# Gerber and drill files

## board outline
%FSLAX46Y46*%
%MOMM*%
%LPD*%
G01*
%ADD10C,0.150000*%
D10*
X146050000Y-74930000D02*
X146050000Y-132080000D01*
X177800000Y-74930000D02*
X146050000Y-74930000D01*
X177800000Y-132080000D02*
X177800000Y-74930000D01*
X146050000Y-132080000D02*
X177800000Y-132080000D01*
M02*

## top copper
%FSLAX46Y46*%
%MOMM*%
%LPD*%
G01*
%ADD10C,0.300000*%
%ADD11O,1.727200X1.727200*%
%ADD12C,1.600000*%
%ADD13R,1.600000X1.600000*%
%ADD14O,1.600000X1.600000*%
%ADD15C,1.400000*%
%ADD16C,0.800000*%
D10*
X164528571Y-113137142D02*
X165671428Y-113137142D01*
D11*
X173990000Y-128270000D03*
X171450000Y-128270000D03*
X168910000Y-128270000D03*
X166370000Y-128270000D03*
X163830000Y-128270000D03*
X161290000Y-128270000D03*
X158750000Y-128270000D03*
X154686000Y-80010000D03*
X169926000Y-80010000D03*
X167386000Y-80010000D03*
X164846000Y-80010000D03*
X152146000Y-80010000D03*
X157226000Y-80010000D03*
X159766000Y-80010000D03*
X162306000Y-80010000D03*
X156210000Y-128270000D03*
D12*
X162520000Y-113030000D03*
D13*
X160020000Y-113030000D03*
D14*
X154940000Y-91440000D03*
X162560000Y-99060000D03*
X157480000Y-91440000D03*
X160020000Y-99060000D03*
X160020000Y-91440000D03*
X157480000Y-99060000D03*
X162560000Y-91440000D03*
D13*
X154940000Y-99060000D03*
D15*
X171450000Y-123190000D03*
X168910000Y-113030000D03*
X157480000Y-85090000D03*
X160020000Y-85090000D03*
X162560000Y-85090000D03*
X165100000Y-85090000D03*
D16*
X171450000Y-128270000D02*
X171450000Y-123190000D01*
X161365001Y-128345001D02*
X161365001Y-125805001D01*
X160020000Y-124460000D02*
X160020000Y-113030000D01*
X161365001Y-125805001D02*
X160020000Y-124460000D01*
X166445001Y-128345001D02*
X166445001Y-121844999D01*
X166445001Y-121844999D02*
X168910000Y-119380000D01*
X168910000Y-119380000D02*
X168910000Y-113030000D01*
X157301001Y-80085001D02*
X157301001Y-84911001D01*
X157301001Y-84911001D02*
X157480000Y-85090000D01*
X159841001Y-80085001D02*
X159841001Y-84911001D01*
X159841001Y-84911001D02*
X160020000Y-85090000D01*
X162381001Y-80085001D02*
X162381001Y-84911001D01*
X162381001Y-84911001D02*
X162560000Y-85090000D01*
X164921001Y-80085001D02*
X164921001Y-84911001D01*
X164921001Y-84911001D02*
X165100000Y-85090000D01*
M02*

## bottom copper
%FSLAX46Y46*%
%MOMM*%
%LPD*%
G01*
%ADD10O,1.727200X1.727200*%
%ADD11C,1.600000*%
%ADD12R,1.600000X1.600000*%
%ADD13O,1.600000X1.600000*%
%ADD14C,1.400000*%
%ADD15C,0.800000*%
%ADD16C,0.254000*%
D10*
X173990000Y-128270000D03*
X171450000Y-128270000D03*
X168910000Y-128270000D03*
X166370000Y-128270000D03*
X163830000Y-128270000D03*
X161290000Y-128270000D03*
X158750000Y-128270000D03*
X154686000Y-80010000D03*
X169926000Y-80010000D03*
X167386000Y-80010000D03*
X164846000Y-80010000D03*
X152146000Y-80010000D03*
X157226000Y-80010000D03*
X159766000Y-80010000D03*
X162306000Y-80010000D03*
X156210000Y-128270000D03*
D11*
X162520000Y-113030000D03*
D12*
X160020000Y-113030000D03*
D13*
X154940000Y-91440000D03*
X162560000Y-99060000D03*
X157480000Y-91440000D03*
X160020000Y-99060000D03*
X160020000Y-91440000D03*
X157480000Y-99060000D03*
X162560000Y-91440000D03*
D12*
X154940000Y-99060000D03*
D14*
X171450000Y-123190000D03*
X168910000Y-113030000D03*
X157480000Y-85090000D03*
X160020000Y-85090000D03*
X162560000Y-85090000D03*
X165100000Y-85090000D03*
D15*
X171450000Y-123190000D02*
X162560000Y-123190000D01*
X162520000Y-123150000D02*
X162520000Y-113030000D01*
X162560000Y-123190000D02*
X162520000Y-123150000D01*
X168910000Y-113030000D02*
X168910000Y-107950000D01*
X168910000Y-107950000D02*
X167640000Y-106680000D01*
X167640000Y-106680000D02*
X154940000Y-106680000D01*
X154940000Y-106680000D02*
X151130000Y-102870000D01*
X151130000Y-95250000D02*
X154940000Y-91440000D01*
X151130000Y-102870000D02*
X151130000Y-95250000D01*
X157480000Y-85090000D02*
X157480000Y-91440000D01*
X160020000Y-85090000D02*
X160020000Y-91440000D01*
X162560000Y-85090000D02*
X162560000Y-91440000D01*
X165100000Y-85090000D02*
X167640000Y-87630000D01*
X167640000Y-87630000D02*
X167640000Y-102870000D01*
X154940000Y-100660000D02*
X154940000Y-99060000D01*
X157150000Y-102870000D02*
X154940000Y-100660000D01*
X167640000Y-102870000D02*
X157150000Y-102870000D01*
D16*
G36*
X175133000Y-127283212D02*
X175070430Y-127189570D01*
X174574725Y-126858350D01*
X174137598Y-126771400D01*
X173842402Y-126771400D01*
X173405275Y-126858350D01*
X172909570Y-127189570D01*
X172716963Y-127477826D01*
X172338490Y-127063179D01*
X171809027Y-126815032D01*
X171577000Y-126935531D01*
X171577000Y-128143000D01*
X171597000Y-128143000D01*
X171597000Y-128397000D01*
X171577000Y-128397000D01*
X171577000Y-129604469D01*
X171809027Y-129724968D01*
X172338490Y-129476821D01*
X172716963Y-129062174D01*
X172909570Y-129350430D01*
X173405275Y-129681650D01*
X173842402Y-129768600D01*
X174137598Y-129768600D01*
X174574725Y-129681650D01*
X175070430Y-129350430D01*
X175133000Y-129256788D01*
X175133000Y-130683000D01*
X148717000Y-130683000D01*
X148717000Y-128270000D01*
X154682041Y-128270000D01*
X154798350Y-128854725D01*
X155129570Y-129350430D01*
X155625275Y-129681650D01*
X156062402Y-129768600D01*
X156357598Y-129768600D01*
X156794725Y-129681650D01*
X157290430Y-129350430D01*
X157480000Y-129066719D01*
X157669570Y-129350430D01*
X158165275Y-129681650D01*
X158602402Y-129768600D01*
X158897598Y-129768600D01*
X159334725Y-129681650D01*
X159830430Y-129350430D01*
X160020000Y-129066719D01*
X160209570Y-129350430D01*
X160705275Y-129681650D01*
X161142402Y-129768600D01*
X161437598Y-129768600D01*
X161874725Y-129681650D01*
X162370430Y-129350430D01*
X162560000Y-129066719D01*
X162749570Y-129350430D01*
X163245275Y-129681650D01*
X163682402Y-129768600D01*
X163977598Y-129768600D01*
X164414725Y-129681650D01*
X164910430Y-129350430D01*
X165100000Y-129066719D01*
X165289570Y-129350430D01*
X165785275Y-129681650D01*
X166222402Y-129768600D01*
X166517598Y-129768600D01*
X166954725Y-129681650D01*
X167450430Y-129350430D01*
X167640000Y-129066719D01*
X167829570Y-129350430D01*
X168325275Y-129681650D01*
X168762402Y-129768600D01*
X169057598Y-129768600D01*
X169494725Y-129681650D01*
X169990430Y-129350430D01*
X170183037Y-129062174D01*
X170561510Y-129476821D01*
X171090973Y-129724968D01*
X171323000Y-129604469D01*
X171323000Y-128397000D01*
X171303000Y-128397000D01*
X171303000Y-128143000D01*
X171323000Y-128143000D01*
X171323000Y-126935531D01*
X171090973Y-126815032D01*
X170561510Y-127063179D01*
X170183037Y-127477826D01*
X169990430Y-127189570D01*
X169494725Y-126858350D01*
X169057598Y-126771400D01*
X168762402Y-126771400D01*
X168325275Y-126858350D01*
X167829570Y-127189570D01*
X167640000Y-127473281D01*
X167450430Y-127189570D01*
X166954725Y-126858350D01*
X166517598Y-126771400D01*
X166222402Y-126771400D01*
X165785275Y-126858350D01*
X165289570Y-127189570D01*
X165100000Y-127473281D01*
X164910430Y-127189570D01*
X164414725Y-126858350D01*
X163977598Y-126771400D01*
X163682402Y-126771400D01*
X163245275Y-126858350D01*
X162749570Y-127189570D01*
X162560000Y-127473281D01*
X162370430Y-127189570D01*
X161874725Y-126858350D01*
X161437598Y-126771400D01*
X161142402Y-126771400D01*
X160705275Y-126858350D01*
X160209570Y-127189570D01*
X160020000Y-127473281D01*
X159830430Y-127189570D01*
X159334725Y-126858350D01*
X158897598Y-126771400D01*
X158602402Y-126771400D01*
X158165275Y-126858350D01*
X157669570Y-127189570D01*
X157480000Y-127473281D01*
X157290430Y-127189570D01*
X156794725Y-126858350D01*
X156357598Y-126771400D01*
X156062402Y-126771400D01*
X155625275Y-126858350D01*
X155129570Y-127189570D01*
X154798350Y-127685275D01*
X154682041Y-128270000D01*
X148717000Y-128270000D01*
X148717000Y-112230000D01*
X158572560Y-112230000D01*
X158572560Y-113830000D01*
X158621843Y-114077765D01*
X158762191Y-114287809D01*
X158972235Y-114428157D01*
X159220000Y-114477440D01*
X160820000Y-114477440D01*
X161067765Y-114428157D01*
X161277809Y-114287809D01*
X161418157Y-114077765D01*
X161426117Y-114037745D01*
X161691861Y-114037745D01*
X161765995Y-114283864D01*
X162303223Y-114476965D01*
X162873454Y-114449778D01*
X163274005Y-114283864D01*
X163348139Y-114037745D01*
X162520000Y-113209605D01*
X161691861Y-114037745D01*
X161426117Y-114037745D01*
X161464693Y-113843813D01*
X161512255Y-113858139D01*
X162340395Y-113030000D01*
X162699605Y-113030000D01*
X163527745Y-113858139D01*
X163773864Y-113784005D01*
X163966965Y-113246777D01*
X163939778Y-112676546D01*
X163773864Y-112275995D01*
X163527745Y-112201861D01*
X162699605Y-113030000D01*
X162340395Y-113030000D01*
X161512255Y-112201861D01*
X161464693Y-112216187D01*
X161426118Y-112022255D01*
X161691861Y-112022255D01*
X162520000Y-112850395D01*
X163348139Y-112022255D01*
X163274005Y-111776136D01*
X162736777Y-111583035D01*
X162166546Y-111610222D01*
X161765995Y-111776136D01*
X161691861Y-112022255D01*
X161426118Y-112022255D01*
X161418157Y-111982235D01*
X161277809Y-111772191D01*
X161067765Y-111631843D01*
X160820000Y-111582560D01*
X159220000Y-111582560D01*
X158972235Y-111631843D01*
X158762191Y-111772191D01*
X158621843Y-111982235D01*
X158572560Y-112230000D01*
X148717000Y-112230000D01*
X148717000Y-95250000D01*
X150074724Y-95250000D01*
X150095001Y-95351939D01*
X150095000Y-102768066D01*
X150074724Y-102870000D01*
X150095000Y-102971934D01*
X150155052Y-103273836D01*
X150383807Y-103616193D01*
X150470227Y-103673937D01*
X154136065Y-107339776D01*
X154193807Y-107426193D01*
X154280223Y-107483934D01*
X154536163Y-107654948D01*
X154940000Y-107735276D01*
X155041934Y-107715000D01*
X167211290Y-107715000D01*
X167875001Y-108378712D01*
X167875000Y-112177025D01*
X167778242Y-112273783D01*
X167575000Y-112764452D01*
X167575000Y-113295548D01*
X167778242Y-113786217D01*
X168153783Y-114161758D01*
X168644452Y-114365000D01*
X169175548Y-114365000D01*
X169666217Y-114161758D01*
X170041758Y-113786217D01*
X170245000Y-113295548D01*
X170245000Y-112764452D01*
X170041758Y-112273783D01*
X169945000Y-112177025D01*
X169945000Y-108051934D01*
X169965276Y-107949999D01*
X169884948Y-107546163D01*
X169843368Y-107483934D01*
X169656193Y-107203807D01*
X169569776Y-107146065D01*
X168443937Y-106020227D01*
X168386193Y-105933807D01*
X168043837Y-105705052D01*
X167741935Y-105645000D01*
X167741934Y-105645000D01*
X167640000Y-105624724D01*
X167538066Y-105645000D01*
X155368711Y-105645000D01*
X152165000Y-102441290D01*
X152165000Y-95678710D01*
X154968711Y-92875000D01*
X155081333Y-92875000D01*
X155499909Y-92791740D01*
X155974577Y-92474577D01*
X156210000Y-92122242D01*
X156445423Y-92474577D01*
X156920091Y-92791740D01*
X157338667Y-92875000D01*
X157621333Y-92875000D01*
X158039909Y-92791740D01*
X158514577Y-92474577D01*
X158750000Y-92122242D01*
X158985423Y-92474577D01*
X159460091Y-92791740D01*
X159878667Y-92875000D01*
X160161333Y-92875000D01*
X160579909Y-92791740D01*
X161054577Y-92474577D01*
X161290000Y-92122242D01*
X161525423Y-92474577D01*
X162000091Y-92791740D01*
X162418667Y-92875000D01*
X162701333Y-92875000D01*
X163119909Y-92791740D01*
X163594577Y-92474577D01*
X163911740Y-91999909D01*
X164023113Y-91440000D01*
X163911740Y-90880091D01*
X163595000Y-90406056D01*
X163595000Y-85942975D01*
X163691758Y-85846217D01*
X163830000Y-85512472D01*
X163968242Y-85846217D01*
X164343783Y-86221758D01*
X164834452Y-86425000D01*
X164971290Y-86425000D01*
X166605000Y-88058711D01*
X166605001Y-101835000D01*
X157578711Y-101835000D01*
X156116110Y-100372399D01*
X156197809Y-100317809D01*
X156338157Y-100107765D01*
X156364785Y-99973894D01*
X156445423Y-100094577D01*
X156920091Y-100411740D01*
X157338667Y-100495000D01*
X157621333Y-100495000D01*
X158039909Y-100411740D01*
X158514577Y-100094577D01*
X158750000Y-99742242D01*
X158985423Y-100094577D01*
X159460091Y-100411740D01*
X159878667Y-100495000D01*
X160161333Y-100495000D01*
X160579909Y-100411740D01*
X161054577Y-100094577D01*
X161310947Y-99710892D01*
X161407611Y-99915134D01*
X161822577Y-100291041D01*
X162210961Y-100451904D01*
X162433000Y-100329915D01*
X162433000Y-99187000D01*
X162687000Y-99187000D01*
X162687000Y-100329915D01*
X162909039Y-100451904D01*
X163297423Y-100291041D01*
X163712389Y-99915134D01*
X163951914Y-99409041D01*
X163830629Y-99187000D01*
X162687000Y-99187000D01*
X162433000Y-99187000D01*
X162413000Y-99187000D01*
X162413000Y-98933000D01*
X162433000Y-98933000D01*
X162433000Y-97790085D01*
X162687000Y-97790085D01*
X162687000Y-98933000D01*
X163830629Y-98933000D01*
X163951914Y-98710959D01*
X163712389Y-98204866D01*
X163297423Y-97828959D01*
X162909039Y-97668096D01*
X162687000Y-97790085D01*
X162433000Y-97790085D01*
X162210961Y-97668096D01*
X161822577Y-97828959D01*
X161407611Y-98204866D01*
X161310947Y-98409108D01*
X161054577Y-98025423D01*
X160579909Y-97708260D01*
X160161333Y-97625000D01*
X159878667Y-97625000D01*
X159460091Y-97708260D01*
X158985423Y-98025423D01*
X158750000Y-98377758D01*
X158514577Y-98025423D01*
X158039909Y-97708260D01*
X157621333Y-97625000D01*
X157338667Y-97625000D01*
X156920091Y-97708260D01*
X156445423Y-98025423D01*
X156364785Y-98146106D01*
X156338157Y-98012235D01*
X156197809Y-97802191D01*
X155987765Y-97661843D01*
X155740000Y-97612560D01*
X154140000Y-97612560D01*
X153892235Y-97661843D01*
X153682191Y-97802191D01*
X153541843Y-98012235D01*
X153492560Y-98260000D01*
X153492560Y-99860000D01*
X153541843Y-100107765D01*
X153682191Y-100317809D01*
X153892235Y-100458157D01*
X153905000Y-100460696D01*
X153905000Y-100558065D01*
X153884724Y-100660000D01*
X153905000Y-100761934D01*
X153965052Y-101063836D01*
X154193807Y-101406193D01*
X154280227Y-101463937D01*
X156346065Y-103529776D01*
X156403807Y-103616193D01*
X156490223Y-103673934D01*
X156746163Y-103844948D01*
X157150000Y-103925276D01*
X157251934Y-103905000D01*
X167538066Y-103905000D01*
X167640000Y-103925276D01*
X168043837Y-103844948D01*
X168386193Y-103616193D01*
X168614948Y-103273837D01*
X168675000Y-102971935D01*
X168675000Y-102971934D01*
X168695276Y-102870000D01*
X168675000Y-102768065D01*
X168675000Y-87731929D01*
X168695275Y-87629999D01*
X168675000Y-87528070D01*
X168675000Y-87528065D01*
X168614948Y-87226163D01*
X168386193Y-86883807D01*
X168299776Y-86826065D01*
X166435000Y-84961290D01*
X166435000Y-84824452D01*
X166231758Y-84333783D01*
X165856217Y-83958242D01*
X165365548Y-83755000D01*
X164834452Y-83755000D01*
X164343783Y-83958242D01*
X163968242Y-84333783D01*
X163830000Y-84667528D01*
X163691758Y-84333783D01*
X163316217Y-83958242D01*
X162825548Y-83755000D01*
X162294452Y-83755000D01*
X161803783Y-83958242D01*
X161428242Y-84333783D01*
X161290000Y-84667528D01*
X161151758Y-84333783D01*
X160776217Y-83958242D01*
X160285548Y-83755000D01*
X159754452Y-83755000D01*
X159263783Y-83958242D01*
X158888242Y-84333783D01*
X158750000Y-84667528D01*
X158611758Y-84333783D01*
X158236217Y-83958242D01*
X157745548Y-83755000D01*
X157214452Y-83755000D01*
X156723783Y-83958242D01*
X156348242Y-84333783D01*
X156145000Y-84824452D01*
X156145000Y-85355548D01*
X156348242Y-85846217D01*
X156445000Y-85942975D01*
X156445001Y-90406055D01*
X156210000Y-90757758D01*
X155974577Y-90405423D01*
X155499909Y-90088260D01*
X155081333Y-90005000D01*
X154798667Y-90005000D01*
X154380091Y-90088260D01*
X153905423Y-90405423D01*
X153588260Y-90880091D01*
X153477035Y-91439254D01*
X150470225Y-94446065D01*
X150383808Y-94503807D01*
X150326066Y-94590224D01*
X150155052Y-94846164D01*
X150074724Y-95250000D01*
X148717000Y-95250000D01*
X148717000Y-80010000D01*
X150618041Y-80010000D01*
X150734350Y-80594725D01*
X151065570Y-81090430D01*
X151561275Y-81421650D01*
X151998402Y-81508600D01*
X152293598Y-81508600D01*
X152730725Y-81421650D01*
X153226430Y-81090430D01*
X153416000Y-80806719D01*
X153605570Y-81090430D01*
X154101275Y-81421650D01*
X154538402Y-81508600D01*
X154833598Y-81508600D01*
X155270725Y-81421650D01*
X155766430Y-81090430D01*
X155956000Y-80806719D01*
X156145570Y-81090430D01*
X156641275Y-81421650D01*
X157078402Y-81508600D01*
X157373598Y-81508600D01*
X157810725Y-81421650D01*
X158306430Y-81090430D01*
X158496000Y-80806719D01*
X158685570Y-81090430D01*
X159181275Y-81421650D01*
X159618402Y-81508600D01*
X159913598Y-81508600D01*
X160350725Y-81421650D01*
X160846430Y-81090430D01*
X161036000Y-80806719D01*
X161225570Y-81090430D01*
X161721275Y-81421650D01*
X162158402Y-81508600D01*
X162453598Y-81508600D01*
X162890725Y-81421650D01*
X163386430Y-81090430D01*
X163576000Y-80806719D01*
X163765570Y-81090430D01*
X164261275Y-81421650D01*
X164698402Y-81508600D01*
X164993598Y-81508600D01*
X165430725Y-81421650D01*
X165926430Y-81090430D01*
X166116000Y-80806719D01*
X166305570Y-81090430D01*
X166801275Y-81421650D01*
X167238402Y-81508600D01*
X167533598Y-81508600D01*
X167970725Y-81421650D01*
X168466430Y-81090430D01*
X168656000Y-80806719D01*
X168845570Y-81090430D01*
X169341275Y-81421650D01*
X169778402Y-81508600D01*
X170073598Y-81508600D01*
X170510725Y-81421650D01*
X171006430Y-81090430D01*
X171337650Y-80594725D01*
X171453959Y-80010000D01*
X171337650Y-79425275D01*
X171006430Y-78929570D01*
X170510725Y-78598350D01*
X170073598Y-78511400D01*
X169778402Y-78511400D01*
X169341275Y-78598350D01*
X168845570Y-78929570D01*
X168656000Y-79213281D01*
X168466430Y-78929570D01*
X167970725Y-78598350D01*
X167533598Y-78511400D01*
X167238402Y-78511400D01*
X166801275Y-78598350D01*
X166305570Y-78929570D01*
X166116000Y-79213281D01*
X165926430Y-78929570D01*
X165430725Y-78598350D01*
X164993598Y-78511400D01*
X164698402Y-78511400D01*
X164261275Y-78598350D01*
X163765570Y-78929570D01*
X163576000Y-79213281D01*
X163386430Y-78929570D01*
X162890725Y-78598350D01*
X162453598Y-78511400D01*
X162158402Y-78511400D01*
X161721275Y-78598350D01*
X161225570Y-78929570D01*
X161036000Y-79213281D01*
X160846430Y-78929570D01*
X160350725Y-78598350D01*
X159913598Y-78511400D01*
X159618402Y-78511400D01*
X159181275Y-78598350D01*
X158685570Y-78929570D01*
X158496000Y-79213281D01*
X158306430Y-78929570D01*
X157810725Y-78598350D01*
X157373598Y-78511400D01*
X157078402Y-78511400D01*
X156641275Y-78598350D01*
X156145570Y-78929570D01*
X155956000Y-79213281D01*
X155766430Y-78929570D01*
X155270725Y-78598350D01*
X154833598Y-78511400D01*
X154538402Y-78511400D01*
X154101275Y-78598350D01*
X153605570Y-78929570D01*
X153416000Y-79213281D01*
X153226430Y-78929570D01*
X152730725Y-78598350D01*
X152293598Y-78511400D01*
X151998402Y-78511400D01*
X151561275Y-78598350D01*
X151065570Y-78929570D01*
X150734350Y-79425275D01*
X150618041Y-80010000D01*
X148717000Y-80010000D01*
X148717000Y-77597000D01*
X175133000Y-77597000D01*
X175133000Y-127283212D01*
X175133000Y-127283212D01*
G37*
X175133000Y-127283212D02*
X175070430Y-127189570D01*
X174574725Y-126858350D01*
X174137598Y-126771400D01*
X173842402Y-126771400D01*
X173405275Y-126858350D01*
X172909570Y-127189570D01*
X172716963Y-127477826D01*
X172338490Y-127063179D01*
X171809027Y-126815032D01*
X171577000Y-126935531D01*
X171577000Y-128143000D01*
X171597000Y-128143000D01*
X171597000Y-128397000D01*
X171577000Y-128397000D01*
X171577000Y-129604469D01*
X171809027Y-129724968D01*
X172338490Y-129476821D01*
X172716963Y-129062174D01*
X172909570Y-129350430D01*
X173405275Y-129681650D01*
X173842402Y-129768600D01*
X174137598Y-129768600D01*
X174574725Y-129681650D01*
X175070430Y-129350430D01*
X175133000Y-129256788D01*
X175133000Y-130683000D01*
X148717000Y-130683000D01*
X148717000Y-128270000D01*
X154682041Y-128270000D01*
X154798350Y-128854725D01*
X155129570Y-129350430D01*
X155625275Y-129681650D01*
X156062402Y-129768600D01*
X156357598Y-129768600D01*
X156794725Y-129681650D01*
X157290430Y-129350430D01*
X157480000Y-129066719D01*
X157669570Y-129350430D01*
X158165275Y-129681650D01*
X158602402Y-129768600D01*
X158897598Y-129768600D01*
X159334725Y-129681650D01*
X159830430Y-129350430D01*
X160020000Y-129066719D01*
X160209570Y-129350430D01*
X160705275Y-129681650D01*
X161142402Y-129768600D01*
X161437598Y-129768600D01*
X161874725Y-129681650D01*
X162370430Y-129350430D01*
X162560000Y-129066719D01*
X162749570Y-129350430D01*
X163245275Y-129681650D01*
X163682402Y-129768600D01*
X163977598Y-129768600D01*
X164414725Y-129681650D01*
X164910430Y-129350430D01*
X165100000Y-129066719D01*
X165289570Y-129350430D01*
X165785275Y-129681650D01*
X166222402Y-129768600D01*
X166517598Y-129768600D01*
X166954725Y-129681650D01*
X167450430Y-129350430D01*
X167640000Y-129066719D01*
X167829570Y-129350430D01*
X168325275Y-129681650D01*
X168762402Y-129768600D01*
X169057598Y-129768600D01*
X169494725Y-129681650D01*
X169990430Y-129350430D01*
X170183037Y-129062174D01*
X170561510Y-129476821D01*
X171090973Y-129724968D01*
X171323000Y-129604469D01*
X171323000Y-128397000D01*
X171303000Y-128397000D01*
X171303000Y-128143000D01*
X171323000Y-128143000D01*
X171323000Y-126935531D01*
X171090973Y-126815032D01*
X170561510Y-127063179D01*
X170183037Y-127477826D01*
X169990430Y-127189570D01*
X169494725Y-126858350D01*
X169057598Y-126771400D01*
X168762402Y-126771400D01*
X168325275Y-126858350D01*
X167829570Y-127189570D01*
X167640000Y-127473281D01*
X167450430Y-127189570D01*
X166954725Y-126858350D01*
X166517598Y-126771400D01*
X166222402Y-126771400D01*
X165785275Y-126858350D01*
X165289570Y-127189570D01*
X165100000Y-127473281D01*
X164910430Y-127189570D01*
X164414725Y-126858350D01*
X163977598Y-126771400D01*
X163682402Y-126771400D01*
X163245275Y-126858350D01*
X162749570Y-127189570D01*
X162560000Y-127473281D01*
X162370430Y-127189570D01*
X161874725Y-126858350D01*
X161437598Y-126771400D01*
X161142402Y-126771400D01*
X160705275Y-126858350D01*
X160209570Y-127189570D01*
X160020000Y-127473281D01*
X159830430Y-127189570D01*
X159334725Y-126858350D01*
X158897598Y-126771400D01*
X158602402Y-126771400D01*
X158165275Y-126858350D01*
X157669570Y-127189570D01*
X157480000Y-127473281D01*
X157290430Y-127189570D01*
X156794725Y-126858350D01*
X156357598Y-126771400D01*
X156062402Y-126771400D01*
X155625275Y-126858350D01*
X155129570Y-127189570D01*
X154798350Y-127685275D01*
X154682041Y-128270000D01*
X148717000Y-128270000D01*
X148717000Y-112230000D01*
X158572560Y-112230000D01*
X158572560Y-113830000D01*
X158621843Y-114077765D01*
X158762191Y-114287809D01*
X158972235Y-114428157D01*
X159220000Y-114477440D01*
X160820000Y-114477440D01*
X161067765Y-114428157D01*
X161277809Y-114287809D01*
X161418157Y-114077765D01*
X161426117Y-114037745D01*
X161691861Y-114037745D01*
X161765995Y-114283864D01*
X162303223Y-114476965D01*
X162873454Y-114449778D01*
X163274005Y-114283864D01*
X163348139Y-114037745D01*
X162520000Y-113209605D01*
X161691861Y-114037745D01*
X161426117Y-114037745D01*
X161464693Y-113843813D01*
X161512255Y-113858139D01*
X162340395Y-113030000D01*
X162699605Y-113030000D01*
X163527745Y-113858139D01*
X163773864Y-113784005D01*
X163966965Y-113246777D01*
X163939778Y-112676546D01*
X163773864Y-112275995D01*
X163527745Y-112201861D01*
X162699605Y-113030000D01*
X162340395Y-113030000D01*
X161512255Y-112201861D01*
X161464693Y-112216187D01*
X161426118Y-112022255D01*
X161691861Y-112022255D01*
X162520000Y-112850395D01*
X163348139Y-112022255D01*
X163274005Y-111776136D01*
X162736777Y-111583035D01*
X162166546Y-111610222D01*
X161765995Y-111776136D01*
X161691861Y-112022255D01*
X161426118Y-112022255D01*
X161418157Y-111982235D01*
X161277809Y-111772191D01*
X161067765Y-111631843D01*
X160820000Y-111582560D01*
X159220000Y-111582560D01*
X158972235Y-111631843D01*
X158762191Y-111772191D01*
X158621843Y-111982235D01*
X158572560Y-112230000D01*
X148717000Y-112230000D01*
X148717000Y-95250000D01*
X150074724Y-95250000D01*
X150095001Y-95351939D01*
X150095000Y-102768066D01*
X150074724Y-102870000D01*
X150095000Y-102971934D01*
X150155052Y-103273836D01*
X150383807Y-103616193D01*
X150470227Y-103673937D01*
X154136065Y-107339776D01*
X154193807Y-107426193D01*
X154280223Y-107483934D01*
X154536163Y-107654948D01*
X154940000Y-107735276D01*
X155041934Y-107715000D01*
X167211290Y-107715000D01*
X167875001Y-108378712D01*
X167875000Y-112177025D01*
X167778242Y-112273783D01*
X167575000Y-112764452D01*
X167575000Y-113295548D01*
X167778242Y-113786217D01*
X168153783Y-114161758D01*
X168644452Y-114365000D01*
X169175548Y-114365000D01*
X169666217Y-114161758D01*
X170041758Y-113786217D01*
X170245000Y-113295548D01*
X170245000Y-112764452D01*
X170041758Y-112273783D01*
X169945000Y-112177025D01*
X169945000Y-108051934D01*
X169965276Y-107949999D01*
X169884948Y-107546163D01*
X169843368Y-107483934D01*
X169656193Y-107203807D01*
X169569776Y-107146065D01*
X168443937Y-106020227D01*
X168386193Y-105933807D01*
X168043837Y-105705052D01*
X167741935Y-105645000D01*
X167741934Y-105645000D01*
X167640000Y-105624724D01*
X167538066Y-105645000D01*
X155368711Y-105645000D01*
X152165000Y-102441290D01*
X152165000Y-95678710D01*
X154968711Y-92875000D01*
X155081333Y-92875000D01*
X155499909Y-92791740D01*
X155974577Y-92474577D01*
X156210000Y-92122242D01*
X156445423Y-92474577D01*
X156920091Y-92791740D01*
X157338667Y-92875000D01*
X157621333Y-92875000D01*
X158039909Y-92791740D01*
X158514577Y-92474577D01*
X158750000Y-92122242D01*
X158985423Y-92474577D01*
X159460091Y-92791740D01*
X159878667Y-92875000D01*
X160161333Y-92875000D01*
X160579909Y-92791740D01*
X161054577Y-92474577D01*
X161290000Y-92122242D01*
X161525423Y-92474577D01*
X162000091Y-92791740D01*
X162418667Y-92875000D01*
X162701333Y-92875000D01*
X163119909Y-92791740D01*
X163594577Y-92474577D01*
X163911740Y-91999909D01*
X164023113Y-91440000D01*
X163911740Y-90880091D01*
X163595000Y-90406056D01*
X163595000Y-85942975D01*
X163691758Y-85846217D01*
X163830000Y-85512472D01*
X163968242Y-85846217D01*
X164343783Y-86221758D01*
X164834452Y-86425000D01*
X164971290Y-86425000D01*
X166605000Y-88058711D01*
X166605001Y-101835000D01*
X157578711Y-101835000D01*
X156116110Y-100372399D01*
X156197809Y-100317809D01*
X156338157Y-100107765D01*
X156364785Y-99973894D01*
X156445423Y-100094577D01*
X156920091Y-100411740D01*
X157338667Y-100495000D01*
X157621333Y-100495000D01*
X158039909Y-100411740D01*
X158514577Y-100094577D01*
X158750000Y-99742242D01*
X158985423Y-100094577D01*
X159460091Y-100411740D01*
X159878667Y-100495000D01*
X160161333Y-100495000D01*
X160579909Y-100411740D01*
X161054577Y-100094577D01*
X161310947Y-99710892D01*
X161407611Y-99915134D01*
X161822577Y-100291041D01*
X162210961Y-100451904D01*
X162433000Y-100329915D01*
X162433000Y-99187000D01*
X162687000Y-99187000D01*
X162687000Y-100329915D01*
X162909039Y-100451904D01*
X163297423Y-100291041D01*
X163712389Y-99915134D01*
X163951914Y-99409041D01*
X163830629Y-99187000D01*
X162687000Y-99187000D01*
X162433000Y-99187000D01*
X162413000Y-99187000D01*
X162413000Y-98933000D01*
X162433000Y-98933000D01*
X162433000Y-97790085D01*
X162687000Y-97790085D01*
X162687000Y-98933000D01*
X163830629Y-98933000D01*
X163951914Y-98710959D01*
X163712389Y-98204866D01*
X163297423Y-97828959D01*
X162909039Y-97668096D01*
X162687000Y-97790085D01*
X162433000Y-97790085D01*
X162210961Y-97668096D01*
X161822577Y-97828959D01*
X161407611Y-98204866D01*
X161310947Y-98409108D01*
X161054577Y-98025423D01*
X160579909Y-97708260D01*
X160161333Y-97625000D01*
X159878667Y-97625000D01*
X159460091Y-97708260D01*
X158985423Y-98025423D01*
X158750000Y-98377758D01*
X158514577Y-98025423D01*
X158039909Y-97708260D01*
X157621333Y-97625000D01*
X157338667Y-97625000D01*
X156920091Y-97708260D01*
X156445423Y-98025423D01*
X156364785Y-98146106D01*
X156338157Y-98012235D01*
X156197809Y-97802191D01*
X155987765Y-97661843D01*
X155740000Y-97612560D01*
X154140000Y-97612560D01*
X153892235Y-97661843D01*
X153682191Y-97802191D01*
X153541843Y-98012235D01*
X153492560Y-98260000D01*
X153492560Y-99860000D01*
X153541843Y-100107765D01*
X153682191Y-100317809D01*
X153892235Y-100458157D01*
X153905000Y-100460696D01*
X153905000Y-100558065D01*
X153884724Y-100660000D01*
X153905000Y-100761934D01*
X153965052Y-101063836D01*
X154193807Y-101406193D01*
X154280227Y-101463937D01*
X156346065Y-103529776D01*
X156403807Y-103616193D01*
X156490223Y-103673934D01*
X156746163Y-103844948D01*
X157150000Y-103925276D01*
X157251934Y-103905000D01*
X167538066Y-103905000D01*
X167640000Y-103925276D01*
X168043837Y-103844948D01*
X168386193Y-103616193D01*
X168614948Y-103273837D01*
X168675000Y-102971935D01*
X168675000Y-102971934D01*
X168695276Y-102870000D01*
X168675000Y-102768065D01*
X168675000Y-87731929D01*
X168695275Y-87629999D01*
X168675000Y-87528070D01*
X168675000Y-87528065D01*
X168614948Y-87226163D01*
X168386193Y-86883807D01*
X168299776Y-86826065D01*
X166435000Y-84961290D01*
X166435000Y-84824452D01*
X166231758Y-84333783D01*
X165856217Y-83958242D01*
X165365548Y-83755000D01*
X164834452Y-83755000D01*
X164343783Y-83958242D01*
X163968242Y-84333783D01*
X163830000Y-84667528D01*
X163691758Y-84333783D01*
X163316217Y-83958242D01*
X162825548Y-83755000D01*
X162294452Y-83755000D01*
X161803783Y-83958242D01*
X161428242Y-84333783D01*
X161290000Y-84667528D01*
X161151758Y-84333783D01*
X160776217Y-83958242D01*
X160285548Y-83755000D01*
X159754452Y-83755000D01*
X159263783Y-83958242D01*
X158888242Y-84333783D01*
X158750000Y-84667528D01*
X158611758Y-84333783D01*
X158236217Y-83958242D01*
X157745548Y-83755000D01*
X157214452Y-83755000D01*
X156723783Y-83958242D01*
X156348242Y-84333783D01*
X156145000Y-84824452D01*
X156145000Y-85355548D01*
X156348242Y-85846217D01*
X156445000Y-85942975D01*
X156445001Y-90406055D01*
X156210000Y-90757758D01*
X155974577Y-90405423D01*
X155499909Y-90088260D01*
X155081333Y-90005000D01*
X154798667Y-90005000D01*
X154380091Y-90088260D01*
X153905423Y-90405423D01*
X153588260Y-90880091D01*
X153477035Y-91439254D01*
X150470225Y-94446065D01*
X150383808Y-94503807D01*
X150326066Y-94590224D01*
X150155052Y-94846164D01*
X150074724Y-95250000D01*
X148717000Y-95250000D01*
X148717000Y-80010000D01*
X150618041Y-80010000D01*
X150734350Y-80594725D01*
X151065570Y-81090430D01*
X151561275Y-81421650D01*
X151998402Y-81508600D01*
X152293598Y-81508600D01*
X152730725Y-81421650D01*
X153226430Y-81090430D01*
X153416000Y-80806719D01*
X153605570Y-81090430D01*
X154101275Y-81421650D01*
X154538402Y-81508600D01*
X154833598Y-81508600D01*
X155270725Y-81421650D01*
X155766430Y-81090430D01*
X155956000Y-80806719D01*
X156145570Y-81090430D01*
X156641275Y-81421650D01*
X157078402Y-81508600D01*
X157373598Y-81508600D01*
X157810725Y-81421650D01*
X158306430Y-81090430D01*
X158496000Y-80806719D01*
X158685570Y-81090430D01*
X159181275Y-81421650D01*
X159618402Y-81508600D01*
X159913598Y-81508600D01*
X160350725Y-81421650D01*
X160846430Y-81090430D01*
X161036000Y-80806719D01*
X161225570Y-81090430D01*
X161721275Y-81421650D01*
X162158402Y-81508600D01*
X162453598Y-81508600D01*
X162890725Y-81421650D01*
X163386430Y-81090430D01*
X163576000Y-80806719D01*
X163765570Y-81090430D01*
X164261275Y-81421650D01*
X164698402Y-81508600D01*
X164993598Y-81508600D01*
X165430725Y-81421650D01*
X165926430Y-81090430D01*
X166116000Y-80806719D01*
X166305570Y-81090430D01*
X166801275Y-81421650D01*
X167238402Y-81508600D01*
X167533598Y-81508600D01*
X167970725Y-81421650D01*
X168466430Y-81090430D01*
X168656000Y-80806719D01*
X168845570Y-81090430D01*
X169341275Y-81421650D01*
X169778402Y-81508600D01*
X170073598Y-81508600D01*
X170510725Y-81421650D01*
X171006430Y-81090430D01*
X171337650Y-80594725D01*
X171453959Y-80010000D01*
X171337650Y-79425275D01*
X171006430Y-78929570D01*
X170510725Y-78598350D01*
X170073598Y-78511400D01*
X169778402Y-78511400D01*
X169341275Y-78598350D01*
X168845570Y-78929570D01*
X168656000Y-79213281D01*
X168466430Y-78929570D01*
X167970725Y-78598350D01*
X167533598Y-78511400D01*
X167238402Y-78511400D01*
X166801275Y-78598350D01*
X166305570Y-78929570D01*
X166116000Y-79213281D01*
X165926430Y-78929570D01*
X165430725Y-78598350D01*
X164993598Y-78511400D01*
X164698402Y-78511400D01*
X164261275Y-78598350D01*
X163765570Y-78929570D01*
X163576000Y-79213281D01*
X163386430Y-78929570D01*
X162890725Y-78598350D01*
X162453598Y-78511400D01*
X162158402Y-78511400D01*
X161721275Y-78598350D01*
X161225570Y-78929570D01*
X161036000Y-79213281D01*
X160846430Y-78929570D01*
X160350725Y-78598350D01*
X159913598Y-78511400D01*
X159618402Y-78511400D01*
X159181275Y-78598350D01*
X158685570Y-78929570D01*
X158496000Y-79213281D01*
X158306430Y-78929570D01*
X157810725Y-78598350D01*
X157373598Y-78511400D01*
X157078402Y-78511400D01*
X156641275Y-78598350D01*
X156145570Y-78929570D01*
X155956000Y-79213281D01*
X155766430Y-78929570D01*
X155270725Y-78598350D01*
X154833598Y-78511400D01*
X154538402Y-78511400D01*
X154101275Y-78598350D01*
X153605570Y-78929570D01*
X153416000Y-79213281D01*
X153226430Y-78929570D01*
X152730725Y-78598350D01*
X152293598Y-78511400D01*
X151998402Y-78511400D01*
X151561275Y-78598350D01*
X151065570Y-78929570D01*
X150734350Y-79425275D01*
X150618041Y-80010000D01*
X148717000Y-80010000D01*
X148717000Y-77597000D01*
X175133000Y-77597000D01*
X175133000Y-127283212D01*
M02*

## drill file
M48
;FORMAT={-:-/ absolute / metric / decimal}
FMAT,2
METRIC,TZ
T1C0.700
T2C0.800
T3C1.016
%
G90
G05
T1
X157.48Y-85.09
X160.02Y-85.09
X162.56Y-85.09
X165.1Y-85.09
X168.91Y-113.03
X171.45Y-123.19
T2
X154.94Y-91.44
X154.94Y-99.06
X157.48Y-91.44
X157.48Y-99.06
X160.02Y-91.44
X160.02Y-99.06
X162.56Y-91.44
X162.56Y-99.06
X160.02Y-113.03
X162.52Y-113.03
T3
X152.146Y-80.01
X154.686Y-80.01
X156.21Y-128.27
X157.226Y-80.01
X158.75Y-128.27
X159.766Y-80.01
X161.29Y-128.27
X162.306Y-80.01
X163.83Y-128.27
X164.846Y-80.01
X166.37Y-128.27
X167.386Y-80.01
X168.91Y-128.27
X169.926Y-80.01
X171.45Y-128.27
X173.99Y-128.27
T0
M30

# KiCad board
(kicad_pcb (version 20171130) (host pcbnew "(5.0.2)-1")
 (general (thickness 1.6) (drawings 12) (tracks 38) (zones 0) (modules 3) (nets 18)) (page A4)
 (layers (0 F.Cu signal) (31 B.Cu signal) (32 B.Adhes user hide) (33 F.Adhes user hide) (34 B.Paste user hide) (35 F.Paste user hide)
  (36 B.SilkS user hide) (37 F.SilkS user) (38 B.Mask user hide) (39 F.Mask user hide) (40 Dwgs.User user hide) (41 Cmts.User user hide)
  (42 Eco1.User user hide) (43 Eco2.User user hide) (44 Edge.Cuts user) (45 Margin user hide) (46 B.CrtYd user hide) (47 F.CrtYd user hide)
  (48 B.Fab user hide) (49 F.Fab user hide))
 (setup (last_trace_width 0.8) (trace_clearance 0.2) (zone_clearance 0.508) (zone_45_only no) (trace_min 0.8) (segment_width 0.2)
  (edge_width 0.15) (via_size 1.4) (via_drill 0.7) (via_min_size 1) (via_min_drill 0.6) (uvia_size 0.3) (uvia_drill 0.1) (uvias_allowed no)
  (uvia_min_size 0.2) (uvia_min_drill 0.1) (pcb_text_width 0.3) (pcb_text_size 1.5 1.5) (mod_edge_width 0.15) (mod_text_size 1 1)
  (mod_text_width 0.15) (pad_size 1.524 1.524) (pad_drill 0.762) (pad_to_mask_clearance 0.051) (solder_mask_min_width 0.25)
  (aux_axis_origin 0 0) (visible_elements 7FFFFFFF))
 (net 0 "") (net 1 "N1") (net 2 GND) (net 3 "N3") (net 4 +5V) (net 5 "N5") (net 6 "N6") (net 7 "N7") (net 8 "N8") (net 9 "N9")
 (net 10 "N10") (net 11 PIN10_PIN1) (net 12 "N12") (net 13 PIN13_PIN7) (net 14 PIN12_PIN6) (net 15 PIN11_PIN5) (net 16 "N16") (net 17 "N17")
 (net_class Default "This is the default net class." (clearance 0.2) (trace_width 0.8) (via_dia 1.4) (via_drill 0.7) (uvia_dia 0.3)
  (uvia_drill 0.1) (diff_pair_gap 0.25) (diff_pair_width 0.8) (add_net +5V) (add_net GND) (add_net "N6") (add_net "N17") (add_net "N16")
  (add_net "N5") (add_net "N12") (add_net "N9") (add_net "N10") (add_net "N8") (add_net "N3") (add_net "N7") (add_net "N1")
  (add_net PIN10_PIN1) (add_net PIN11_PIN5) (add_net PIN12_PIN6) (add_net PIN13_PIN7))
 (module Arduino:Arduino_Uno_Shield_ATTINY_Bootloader (layer F.Cu) (at 128.27 130.81)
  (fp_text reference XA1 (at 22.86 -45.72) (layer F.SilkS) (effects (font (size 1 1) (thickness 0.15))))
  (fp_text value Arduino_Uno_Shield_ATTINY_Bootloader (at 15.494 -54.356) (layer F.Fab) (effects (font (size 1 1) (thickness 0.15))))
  (pad VIN thru_hole oval (at 45.72 -2.54) (size 1.7272 1.7272) (drill 1.016) (layers *.Cu *.Mask) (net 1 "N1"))
  (pad GND3 thru_hole oval (at 43.18 -2.54) (size 1.7272 1.7272) (drill 1.016) (layers *.Cu *.Mask) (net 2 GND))
  (pad GND2 thru_hole oval (at 40.64 -2.54) (size 1.7272 1.7272) (drill 1.016) (layers *.Cu *.Mask) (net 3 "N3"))
  (pad 5V1 thru_hole oval (at 38.1 -2.54) (size 1.7272 1.7272) (drill 1.016) (layers *.Cu *.Mask) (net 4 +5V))
  (pad 3V3 thru_hole oval (at 35.56 -2.54) (size 1.7272 1.7272) (drill 1.016) (layers *.Cu *.Mask) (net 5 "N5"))
  (pad RST1 thru_hole oval (at 33.02 -2.54) (size 1.7272 1.7272) (drill 1.016) (layers *.Cu *.Mask) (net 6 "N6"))
  (pad IORF thru_hole oval (at 30.48 -2.54) (size 1.7272 1.7272) (drill 1.016) (layers *.Cu *.Mask) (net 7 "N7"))
  (pad GND1 thru_hole oval (at 26.416 -50.8) (size 1.7272 1.7272) (drill 1.016) (layers *.Cu *.Mask) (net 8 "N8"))
  (pad D8 thru_hole oval (at 41.656 -50.8) (size 1.7272 1.7272) (drill 1.016) (layers *.Cu *.Mask) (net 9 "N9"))
  (pad D9 thru_hole oval (at 39.116 -50.8) (size 1.7272 1.7272) (drill 1.016) (layers *.Cu *.Mask) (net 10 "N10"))
  (pad D10 thru_hole oval (at 36.576 -50.8) (size 1.7272 1.7272) (drill 1.016) (layers *.Cu *.Mask) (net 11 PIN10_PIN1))
  (pad AREF thru_hole oval (at 23.876 -50.8) (size 1.7272 1.7272) (drill 1.016) (layers *.Cu *.Mask) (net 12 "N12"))
  (pad D13 thru_hole oval (at 28.956 -50.8) (size 1.7272 1.7272) (drill 1.016) (layers *.Cu *.Mask) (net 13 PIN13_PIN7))
  (pad D12 thru_hole oval (at 31.496 -50.8) (size 1.7272 1.7272) (drill 1.016) (layers *.Cu *.Mask) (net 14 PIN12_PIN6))
  (pad D11 thru_hole oval (at 34.036 -50.8) (size 1.7272 1.7272) (drill 1.016) (layers *.Cu *.Mask) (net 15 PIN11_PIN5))
  (pad "" thru_hole oval (at 27.94 -2.54) (size 1.7272 1.7272) (drill 1.016) (layers *.Cu *.Mask)))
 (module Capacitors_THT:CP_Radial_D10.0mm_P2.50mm (layer F.Cu) (at 160.02 113.03)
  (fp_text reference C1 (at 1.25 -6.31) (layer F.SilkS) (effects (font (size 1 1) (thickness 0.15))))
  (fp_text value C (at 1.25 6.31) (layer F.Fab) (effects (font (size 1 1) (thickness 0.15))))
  (pad 2 thru_hole circle (at 2.5 0) (size 1.6 1.6) (drill 0.8) (layers *.Cu *.Mask) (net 2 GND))
  (pad 1 thru_hole rect (at 0 0) (size 1.6 1.6) (drill 0.8) (layers *.Cu *.Mask) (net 6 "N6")))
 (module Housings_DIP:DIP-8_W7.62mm (layer F.Cu) (at 154.94 99.06 90)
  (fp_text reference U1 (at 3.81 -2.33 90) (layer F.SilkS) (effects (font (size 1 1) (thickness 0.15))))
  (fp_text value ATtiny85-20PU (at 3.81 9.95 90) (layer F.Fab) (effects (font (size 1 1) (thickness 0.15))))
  (pad 8 thru_hole oval (at 7.62 0 90) (size 1.6 1.6) (drill 0.8) (layers *.Cu *.Mask) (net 4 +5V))
  (pad 4 thru_hole oval (at 0 7.62 90) (size 1.6 1.6) (drill 0.8) (layers *.Cu *.Mask) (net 2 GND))
  (pad 7 thru_hole oval (at 7.62 2.54 90) (size 1.6 1.6) (drill 0.8) (layers *.Cu *.Mask) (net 13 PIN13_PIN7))
  (pad 3 thru_hole oval (at 0 5.08 90) (size 1.6 1.6) (drill 0.8) (layers *.Cu *.Mask) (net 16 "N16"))
  (pad 6 thru_hole oval (at 7.62 5.08 90) (size 1.6 1.6) (drill 0.8) (layers *.Cu *.Mask) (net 14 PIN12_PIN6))
  (pad 2 thru_hole oval (at 0 2.54 90) (size 1.6 1.6) (drill 0.8) (layers *.Cu *.Mask) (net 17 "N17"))
  (pad 5 thru_hole oval (at 7.62 7.62 90) (size 1.6 1.6) (drill 0.8) (layers *.Cu *.Mask) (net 15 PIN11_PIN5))
  (pad 1 thru_hole rect (at 0 0 90) (size 1.6 1.6) (drill 0.8) (layers *.Cu *.Mask) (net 11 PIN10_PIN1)))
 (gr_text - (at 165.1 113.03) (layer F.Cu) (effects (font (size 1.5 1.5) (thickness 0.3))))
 (gr_line (start 146.05 74.93) (end 146.05 132.08) (layer Edge.Cuts) (width 0.15))
 (gr_line (start 177.8 74.93) (end 146.05 74.93) (layer Edge.Cuts) (width 0.15))
 (gr_line (start 177.8 132.08) (end 177.8 74.93) (layer Edge.Cuts) (width 0.15))
 (gr_line (start 146.05 132.08) (end 177.8 132.08) (layer Edge.Cuts) (width 0.15))
 (via (at 171.45 123.19) (size 1.4) (drill 0.7) (layers F.Cu B.Cu) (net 2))
 (segment (start 171.45 128.27) (end 171.45 123.19) (width 0.8) (layer F.Cu) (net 2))
 (segment (start 171.45 123.19) (end 162.56 123.19) (width 0.8) (layer B.Cu) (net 2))
 (segment (start 162.52 123.15) (end 162.52 113.03) (width 0.8) (layer B.Cu) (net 2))
 (segment (start 162.56 123.19) (end 162.52 123.15) (width 0.8) (layer B.Cu) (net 2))
 (segment (start 161.365001 128.345001) (end 161.365001 125.805001) (width 0.8) (layer F.Cu) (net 6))
 (segment (start 160.02 124.46) (end 160.02 113.03) (width 0.8) (layer F.Cu) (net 6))
 (segment (start 161.365001 125.805001) (end 160.02 124.46) (width 0.8) (layer F.Cu) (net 6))
 (segment (start 166.445001 128.345001) (end 166.445001 121.844999) (width 0.8) (layer F.Cu) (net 4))
 (via (at 168.91 113.03) (size 1.4) (drill 0.7) (layers F.Cu B.Cu) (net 4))
 (segment (start 166.445001 121.844999) (end 168.91 119.38) (width 0.8) (layer F.Cu) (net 4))
 (segment (start 168.91 119.38) (end 168.91 113.03) (width 0.8) (layer F.Cu) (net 4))
 (segment (start 168.91 113.03) (end 168.91 107.95) (width 0.8) (layer B.Cu) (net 4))
 (segment (start 168.91 107.95) (end 167.64 106.68) (width 0.8) (layer B.Cu) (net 4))
 (segment (start 167.64 106.68) (end 154.94 106.68) (width 0.8) (layer B.Cu) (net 4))
 (segment (start 154.94 106.68) (end 151.13 102.87) (width 0.8) (layer B.Cu) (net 4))
 (segment (start 151.13 95.25) (end 154.94 91.44) (width 0.8) (layer B.Cu) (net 4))
 (segment (start 151.13 102.87) (end 151.13 95.25) (width 0.8) (layer B.Cu) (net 4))
 (via (at 157.48 85.09) (size 1.4) (drill 0.7) (layers F.Cu B.Cu) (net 13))
 (segment (start 157.301001 80.085001) (end 157.301001 84.911001) (width 0.8) (layer F.Cu) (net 13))
 (segment (start 157.301001 84.911001) (end 157.48 85.09) (width 0.8) (layer F.Cu) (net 13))
 (segment (start 157.48 85.09) (end 157.48 91.44) (width 0.8) (layer B.Cu) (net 13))
 (via (at 160.02 85.09) (size 1.4) (drill 0.7) (layers F.Cu B.Cu) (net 14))
 (segment (start 159.841001 80.085001) (end 159.841001 84.911001) (width 0.8) (layer F.Cu) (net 14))
 (segment (start 159.841001 84.911001) (end 160.02 85.09) (width 0.8) (layer F.Cu) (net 14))
 (segment (start 160.02 85.09) (end 160.02 91.44) (width 0.8) (layer B.Cu) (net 14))
 (via (at 162.56 85.09) (size 1.4) (drill 0.7) (layers F.Cu B.Cu) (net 15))
 (segment (start 162.381001 80.085001) (end 162.381001 84.911001) (width 0.8) (layer F.Cu) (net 15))
 (segment (start 162.381001 84.911001) (end 162.56 85.09) (width 0.8) (layer F.Cu) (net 15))
 (segment (start 162.56 85.09) (end 162.56 91.44) (width 0.8) (layer B.Cu) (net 15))
 (via (at 165.1 85.09) (size 1.4) (drill 0.7) (layers F.Cu B.Cu) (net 11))
 (segment (start 164.921001 80.085001) (end 164.921001 84.911001) (width 0.8) (layer F.Cu) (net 11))
 (segment (start 164.921001 84.911001) (end 165.1 85.09) (width 0.8) (layer F.Cu) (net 11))
 (segment (start 165.1 85.09) (end 167.64 87.63) (width 0.8) (layer B.Cu) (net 11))
 (segment (start 167.64 87.63) (end 167.64 102.87) (width 0.8) (layer B.Cu) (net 11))
 (segment (start 154.94 100.66) (end 154.94 99.06) (width 0.8) (layer B.Cu) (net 11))
 (segment (start 157.15 102.87) (end 154.94 100.66) (width 0.8) (layer B.Cu) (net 11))
 (segment (start 167.64 102.87) (end 157.15 102.87) (width 0.8) (layer B.Cu) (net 11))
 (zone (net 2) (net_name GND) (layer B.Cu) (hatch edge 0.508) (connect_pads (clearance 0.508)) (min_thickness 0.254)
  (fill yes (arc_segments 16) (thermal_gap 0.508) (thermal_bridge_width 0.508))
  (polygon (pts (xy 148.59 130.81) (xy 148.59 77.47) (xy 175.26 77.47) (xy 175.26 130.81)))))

